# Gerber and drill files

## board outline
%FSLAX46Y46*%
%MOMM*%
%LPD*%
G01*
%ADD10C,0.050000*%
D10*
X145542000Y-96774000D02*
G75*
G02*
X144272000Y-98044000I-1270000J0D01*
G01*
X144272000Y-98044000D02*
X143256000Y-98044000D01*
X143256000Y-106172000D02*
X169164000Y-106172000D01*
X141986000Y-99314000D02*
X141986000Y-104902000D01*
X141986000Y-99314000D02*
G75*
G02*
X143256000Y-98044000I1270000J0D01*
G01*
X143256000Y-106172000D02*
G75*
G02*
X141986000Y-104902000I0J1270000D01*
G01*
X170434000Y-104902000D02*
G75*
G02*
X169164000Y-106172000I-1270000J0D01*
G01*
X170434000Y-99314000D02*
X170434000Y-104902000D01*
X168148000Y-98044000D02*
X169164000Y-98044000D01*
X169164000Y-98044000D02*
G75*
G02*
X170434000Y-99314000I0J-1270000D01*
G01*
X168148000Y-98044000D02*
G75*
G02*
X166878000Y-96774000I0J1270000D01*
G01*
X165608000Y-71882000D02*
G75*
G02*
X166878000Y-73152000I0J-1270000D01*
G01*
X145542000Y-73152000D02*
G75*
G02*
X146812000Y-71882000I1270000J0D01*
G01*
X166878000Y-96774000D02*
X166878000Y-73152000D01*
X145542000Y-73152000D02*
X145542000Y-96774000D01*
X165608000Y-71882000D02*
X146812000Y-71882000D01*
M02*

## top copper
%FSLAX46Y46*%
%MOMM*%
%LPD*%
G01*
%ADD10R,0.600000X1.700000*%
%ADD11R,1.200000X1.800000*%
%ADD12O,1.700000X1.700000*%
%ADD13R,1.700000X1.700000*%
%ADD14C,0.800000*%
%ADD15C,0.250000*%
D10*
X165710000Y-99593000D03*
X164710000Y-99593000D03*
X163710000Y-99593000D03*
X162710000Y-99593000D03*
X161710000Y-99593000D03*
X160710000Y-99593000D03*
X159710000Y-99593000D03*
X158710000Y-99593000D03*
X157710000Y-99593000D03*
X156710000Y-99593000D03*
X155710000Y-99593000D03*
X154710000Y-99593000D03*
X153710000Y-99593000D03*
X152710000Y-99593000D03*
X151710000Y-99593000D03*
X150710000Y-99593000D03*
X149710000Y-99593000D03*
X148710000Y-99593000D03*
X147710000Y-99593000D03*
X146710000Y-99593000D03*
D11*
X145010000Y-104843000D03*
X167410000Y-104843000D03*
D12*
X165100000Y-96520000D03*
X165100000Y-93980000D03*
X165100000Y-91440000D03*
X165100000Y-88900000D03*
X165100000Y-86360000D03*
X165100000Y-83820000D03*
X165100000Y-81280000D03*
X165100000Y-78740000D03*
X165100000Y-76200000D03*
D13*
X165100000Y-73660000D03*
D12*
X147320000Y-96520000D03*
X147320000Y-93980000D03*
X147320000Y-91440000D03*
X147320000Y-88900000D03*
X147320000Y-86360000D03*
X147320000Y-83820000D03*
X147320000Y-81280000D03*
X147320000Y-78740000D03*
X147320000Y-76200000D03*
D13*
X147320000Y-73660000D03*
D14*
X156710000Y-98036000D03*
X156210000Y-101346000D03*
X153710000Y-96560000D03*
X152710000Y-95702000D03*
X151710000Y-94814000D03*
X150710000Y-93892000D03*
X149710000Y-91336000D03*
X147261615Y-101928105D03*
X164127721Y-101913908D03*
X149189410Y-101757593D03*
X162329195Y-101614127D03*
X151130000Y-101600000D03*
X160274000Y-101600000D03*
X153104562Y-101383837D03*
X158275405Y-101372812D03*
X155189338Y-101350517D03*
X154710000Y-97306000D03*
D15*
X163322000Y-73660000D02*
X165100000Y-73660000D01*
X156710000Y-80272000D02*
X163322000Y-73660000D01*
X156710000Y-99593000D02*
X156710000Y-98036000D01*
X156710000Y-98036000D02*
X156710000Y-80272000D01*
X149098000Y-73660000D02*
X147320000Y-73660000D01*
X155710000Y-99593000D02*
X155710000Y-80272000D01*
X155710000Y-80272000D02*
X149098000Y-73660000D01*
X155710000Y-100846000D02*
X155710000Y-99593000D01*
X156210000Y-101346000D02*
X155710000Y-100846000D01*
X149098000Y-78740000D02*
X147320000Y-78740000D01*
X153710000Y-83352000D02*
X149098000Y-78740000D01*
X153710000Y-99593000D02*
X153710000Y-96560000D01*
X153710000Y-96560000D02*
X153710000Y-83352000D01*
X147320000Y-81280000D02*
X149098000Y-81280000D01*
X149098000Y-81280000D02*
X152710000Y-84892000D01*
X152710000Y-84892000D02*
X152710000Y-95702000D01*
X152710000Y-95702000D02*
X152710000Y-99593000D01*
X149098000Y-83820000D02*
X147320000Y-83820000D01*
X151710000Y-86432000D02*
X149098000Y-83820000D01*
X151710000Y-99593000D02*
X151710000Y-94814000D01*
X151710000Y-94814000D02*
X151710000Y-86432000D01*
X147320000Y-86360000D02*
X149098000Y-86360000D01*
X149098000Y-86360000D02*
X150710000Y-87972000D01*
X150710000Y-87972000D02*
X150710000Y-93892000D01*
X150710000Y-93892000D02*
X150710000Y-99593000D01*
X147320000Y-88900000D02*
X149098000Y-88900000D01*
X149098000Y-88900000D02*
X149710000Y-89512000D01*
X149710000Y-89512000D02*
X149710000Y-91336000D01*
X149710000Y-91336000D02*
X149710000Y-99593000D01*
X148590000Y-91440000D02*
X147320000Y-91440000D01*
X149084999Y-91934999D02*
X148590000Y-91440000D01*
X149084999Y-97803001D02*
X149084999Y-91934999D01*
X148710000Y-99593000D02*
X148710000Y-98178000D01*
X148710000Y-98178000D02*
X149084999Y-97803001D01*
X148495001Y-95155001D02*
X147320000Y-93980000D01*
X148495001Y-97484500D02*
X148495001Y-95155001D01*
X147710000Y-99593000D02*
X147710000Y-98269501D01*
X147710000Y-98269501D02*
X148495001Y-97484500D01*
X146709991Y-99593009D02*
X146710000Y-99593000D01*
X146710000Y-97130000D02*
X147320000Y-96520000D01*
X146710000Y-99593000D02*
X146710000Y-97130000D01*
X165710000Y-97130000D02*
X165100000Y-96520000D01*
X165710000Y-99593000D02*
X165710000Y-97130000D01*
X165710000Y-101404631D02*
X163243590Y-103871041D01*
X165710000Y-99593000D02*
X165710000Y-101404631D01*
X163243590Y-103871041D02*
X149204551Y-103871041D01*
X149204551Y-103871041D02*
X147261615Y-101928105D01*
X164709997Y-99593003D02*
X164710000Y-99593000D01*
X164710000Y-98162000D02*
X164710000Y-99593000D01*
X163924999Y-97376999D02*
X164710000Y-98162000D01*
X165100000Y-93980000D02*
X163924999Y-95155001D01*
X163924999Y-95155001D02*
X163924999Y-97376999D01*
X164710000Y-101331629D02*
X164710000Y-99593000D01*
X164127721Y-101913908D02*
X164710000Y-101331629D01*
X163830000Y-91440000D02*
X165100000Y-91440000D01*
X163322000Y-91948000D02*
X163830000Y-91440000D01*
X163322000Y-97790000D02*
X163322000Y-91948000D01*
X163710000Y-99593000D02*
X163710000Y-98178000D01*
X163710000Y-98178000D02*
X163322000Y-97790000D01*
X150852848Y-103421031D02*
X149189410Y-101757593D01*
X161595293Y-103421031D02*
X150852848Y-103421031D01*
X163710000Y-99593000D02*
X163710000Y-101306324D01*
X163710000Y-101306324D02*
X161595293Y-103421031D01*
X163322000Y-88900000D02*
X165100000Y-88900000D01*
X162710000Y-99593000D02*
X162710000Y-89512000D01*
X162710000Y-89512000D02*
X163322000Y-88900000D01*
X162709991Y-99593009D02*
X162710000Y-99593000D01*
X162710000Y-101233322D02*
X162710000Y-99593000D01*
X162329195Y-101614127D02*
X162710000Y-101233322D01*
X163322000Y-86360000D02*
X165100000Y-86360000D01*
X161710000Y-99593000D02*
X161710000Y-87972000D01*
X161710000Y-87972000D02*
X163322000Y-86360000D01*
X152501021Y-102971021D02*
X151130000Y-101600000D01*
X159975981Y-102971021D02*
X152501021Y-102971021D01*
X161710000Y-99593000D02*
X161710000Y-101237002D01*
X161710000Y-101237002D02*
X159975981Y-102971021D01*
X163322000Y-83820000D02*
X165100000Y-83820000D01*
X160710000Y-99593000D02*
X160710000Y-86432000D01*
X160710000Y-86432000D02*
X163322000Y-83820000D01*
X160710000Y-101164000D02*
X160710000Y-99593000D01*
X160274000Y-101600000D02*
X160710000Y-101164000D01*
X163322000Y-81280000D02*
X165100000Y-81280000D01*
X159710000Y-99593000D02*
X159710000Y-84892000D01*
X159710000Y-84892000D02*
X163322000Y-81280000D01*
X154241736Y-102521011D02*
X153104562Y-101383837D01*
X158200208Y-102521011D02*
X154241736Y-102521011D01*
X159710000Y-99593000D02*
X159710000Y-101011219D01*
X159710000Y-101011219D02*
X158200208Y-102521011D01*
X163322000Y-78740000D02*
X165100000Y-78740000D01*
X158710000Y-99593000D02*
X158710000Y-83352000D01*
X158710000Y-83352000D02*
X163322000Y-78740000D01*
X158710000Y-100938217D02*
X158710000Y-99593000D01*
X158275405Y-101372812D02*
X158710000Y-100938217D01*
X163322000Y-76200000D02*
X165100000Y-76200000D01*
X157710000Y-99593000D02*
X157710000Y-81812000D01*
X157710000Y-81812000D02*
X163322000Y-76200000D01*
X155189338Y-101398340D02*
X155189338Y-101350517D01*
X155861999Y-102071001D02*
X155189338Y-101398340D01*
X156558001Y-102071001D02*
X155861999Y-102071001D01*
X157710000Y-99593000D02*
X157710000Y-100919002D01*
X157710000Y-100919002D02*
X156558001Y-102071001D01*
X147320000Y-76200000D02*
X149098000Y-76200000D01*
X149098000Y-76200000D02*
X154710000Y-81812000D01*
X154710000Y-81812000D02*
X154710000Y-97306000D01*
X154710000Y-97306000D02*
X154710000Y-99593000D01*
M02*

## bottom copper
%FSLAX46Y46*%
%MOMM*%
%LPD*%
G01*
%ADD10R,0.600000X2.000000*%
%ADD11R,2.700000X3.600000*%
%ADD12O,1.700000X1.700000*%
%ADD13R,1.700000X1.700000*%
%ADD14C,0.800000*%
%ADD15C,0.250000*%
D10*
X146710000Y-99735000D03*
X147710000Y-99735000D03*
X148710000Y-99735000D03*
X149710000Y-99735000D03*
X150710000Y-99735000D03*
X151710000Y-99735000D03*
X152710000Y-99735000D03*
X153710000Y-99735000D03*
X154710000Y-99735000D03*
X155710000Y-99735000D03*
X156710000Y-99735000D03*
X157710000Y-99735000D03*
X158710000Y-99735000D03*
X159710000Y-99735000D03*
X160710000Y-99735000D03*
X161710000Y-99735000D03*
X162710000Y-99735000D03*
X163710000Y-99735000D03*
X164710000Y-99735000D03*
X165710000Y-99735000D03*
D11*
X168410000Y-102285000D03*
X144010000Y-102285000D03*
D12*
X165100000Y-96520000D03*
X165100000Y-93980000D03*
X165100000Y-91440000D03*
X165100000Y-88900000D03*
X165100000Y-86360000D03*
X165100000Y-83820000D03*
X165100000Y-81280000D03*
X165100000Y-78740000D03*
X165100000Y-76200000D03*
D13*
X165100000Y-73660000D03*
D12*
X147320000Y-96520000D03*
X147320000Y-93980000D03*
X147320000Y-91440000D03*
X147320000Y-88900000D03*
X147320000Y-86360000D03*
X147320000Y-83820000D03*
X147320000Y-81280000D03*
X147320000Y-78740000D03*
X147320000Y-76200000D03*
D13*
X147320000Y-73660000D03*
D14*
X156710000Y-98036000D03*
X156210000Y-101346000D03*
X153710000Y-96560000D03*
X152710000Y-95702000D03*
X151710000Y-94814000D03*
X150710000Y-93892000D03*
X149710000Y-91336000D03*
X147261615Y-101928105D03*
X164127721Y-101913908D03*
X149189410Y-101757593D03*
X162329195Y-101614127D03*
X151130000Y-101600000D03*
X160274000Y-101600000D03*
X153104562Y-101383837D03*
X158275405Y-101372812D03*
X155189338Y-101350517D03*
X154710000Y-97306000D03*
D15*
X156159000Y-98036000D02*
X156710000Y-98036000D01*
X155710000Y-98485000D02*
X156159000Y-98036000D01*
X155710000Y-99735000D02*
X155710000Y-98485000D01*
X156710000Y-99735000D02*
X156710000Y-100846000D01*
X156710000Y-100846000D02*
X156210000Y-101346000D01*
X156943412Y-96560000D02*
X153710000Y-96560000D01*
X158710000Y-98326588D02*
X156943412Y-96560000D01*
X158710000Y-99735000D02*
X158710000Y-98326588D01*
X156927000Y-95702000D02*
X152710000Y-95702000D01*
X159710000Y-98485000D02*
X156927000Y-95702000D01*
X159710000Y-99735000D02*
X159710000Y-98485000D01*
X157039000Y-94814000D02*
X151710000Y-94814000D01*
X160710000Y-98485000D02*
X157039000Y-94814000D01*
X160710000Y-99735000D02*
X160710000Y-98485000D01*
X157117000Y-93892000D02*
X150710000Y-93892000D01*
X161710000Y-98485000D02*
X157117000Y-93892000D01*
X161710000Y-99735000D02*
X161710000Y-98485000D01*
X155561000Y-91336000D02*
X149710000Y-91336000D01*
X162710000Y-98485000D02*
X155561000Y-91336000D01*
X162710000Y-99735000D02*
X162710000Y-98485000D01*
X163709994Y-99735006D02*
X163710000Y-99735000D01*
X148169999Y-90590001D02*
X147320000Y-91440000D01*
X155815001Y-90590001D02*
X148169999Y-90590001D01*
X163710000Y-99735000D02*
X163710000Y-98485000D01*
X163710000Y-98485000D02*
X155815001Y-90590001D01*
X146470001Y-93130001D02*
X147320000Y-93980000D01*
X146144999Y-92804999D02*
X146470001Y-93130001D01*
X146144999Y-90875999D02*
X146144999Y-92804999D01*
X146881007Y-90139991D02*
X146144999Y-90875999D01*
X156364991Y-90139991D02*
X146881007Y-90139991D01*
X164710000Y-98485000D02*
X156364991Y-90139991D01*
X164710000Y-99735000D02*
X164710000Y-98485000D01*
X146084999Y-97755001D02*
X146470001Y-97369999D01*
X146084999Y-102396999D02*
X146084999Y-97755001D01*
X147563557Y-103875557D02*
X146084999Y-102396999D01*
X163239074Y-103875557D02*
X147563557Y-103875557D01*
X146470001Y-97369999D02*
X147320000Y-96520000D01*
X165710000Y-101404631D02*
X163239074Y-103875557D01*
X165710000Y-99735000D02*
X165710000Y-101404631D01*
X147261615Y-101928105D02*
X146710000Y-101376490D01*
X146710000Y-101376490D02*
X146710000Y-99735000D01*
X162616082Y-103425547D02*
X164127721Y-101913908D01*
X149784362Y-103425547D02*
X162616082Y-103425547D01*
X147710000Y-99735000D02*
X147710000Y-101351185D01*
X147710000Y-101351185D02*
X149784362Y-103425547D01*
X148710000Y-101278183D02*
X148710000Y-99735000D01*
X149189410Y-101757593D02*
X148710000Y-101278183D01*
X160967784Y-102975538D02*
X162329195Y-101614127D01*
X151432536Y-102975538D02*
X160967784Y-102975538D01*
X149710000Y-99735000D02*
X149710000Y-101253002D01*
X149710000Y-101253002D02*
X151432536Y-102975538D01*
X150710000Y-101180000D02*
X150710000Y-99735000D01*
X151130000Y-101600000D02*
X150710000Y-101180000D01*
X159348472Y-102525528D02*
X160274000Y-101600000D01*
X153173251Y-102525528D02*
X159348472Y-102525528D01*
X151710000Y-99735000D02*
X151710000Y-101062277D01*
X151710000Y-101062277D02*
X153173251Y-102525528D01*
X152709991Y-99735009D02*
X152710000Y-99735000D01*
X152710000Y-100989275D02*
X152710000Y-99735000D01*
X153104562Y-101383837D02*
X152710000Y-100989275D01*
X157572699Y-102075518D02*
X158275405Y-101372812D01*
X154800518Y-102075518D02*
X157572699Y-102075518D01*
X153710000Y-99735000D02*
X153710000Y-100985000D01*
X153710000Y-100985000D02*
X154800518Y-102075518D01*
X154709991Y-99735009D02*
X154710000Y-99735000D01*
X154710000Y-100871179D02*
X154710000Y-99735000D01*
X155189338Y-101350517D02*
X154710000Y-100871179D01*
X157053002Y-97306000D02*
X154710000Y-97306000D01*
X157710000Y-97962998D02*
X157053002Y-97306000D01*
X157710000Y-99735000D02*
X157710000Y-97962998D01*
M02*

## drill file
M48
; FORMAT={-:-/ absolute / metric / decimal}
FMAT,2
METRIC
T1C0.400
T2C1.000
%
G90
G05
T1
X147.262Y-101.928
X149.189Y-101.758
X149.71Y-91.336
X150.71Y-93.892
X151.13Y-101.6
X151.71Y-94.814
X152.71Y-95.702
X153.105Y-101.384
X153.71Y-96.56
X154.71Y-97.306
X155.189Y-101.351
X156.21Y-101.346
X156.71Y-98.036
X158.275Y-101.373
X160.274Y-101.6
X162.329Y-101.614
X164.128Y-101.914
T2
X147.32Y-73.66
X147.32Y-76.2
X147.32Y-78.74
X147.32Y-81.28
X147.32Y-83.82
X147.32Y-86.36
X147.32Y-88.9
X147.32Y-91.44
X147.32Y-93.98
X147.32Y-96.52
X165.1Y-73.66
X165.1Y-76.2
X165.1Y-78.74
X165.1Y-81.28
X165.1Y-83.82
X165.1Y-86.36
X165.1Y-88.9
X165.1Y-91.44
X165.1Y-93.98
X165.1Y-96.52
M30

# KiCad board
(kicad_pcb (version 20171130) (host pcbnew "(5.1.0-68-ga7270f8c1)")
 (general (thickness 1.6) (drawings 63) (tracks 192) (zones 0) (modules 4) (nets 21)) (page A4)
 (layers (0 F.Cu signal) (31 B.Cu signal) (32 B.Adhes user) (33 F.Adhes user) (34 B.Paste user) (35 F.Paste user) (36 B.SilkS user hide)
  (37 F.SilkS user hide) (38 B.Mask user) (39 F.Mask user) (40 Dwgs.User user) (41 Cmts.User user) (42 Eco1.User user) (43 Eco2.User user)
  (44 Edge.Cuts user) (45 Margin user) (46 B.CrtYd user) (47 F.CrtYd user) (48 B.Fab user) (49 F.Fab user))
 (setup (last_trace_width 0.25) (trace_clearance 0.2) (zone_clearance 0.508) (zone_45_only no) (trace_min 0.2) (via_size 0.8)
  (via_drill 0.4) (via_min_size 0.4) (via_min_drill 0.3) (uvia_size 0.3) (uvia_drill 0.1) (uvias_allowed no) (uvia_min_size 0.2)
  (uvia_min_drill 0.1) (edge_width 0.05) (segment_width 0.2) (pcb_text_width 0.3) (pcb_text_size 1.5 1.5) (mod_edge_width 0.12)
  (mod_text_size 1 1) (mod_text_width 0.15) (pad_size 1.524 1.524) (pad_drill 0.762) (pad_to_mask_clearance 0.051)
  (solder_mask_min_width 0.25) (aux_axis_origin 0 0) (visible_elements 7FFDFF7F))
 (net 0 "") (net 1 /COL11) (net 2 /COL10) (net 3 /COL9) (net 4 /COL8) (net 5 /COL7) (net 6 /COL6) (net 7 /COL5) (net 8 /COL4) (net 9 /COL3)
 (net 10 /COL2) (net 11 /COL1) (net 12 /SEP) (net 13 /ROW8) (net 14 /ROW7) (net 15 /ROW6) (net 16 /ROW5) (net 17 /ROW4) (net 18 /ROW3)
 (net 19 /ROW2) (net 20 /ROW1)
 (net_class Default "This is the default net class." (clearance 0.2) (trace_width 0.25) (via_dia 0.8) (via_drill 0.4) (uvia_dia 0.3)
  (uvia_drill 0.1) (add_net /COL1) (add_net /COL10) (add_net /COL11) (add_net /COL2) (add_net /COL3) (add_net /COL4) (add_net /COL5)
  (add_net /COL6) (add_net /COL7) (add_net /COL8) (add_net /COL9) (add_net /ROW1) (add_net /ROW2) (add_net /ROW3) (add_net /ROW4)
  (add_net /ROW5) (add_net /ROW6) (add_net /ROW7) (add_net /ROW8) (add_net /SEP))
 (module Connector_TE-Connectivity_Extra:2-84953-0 (layer B.Cu) (at 156.21 101.635 180)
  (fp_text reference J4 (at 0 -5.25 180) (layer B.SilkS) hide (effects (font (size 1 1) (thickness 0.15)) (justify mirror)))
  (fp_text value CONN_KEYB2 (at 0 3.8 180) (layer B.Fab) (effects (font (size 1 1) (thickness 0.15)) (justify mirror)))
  (pad 20 smd rect (at 9.5 1.9 180) (size 0.6 2) (layers B.Cu B.Paste B.Mask) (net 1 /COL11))
  (pad 19 smd rect (at 8.5 1.9 180) (size 0.6 2) (layers B.Cu B.Paste B.Mask) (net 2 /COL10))
  (pad 18 smd rect (at 7.5 1.9 180) (size 0.6 2) (layers B.Cu B.Paste B.Mask) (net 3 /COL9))
  (pad 17 smd rect (at 6.5 1.9 180) (size 0.6 2) (layers B.Cu B.Paste B.Mask) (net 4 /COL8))
  (pad 16 smd rect (at 5.5 1.9 180) (size 0.6 2) (layers B.Cu B.Paste B.Mask) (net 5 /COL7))
  (pad 15 smd rect (at 4.5 1.9 180) (size 0.6 2) (layers B.Cu B.Paste B.Mask) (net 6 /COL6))
  (pad 14 smd rect (at 3.5 1.9 180) (size 0.6 2) (layers B.Cu B.Paste B.Mask) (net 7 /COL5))
  (pad 13 smd rect (at 2.5 1.9 180) (size 0.6 2) (layers B.Cu B.Paste B.Mask) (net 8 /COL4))
  (pad 12 smd rect (at 1.5 1.9 180) (size 0.6 2) (layers B.Cu B.Paste B.Mask) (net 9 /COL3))
  (pad 11 smd rect (at 0.5 1.9 180) (size 0.6 2) (layers B.Cu B.Paste B.Mask) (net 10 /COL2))
  (pad 10 smd rect (at -0.5 1.9 180) (size 0.6 2) (layers B.Cu B.Paste B.Mask) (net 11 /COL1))
  (pad 9 smd rect (at -1.5 1.9 180) (size 0.6 2) (layers B.Cu B.Paste B.Mask) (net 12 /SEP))
  (pad 8 smd rect (at -2.5 1.9 180) (size 0.6 2) (layers B.Cu B.Paste B.Mask) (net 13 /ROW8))
  (pad 7 smd rect (at -3.5 1.9 180) (size 0.6 2) (layers B.Cu B.Paste B.Mask) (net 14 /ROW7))
  (pad 6 smd rect (at -4.5 1.9 180) (size 0.6 2) (layers B.Cu B.Paste B.Mask) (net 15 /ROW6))
  (pad 5 smd rect (at -5.5 1.9 180) (size 0.6 2) (layers B.Cu B.Paste B.Mask) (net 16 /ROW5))
  (pad 4 smd rect (at -6.5 1.9 180) (size 0.6 2) (layers B.Cu B.Paste B.Mask) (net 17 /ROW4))
  (pad 3 smd rect (at -7.5 1.9 180) (size 0.6 2) (layers B.Cu B.Paste B.Mask) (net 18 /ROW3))
  (pad 2 smd rect (at -8.5 1.9 180) (size 0.6 2) (layers B.Cu B.Paste B.Mask) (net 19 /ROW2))
  (pad 1 smd rect (at -9.5 1.9 180) (size 0.6 2) (layers B.Cu B.Paste B.Mask) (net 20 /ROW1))
  (pad "" smd rect (at -12.2 -0.65 180) (size 2.7 3.6) (layers B.Cu B.Paste B.Mask))
  (pad "" smd rect (at 12.2 -0.65 180) (size 2.7 3.6) (layers B.Cu B.Paste B.Mask)))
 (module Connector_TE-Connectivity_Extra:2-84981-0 (layer F.Cu) (at 156.21 102.743)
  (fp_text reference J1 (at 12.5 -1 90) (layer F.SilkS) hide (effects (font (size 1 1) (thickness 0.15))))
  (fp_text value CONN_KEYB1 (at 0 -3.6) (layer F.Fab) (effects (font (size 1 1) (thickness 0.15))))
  (pad 20 smd rect (at 9.5 -3.15) (size 0.6 1.7) (layers F.Cu F.Paste F.Mask) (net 1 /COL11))
  (pad 19 smd rect (at 8.5 -3.15) (size 0.6 1.7) (layers F.Cu F.Paste F.Mask) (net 2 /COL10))
  (pad 18 smd rect (at 7.5 -3.15) (size 0.6 1.7) (layers F.Cu F.Paste F.Mask) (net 3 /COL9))
  (pad 17 smd rect (at 6.5 -3.15) (size 0.6 1.7) (layers F.Cu F.Paste F.Mask) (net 4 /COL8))
  (pad 16 smd rect (at 5.5 -3.15) (size 0.6 1.7) (layers F.Cu F.Paste F.Mask) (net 5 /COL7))
  (pad 15 smd rect (at 4.5 -3.15) (size 0.6 1.7) (layers F.Cu F.Paste F.Mask) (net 6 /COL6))
  (pad 14 smd rect (at 3.5 -3.15) (size 0.6 1.7) (layers F.Cu F.Paste F.Mask) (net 7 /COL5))
  (pad 13 smd rect (at 2.5 -3.15) (size 0.6 1.7) (layers F.Cu F.Paste F.Mask) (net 8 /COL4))
  (pad 12 smd rect (at 1.5 -3.15) (size 0.6 1.7) (layers F.Cu F.Paste F.Mask) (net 9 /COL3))
  (pad 11 smd rect (at 0.5 -3.15) (size 0.6 1.7) (layers F.Cu F.Paste F.Mask) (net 10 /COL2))
  (pad 10 smd rect (at -0.5 -3.15) (size 0.6 1.7) (layers F.Cu F.Paste F.Mask) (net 11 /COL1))
  (pad 9 smd rect (at -1.5 -3.15) (size 0.6 1.7) (layers F.Cu F.Paste F.Mask) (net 12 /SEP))
  (pad 8 smd rect (at -2.5 -3.15) (size 0.6 1.7) (layers F.Cu F.Paste F.Mask) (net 13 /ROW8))
  (pad 7 smd rect (at -3.5 -3.15) (size 0.6 1.7) (layers F.Cu F.Paste F.Mask) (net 14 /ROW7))
  (pad 6 smd rect (at -4.5 -3.15) (size 0.6 1.7) (layers F.Cu F.Paste F.Mask) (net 15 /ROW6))
  (pad 5 smd rect (at -5.5 -3.15) (size 0.6 1.7) (layers F.Cu F.Paste F.Mask) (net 16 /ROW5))
  (pad 4 smd rect (at -6.5 -3.15) (size 0.6 1.7) (layers F.Cu F.Paste F.Mask) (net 17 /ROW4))
  (pad 3 smd rect (at -7.5 -3.15) (size 0.6 1.7) (layers F.Cu F.Paste F.Mask) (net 18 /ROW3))
  (pad 2 smd rect (at -8.5 -3.15) (size 0.6 1.7) (layers F.Cu F.Paste F.Mask) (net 19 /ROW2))
  (pad 1 smd rect (at -9.5 -3.15) (size 0.6 1.7) (layers F.Cu F.Paste F.Mask) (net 20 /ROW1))
  (pad "" smd rect (at -11.2 2.1) (size 1.2 1.8) (layers F.Cu F.Paste F.Mask))
  (pad "" smd rect (at 11.2 2.1) (size 1.2 1.8) (layers F.Cu F.Paste F.Mask)))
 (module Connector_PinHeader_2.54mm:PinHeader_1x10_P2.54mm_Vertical (layer F.Cu) (at 165.1 73.66)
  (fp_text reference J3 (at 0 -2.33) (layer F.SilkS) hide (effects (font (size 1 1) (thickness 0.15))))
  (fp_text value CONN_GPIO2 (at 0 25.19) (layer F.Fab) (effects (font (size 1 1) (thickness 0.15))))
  (pad 10 thru_hole oval (at 0 22.86) (size 1.7 1.7) (drill 1) (layers *.Cu *.Mask) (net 1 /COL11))
  (pad 9 thru_hole oval (at 0 20.32) (size 1.7 1.7) (drill 1) (layers *.Cu *.Mask) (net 2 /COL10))
  (pad 8 thru_hole oval (at 0 17.78) (size 1.7 1.7) (drill 1) (layers *.Cu *.Mask) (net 3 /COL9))
  (pad 7 thru_hole oval (at 0 15.24) (size 1.7 1.7) (drill 1) (layers *.Cu *.Mask) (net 4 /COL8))
  (pad 6 thru_hole oval (at 0 12.7) (size 1.7 1.7) (drill 1) (layers *.Cu *.Mask) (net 5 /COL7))
  (pad 5 thru_hole oval (at 0 10.16) (size 1.7 1.7) (drill 1) (layers *.Cu *.Mask) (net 6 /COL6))
  (pad 4 thru_hole oval (at 0 7.62) (size 1.7 1.7) (drill 1) (layers *.Cu *.Mask) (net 7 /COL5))
  (pad 3 thru_hole oval (at 0 5.08) (size 1.7 1.7) (drill 1) (layers *.Cu *.Mask) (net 8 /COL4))
  (pad 2 thru_hole oval (at 0 2.54) (size 1.7 1.7) (drill 1) (layers *.Cu *.Mask) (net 9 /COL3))
  (pad 1 thru_hole rect (at 0 0) (size 1.7 1.7) (drill 1) (layers *.Cu *.Mask) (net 10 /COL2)))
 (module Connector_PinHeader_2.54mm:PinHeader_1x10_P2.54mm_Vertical (layer F.Cu) (at 147.32 73.66)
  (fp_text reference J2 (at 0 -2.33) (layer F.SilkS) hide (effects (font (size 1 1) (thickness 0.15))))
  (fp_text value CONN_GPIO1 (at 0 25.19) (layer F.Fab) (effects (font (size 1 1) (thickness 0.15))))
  (pad 10 thru_hole oval (at 0 22.86) (size 1.7 1.7) (drill 1) (layers *.Cu *.Mask) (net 20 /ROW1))
  (pad 9 thru_hole oval (at 0 20.32) (size 1.7 1.7) (drill 1) (layers *.Cu *.Mask) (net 19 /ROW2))
  (pad 8 thru_hole oval (at 0 17.78) (size 1.7 1.7) (drill 1) (layers *.Cu *.Mask) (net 18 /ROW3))
  (pad 7 thru_hole oval (at 0 15.24) (size 1.7 1.7) (drill 1) (layers *.Cu *.Mask) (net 17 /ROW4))
  (pad 6 thru_hole oval (at 0 12.7) (size 1.7 1.7) (drill 1) (layers *.Cu *.Mask) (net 16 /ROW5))
  (pad 5 thru_hole oval (at 0 10.16) (size 1.7 1.7) (drill 1) (layers *.Cu *.Mask) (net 15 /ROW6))
  (pad 4 thru_hole oval (at 0 7.62) (size 1.7 1.7) (drill 1) (layers *.Cu *.Mask) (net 14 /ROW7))
  (pad 3 thru_hole oval (at 0 5.08) (size 1.7 1.7) (drill 1) (layers *.Cu *.Mask) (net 13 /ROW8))
  (pad 2 thru_hole oval (at 0 2.54) (size 1.7 1.7) (drill 1) (layers *.Cu *.Mask) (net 12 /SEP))
  (pad 1 thru_hole rect (at 0 0) (size 1.7 1.7) (drill 1) (layers *.Cu *.Mask) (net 11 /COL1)))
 (gr_arc (start 144.272 96.774) (end 144.272 98.044) (angle -90) (layer Edge.Cuts) (width 0.05))
 (gr_line (start 144.272 98.044) (end 143.256 98.044) (layer Edge.Cuts) (width 0.05))
 (gr_line (start 143.256 106.172) (end 169.164 106.172) (layer Edge.Cuts) (width 0.05))
 (gr_line (start 141.986 99.314) (end 141.986 104.902) (layer Edge.Cuts) (width 0.05))
 (gr_arc (start 143.256 99.314) (end 143.256 98.044) (angle -90) (layer Edge.Cuts) (width 0.05))
 (gr_arc (start 143.256 104.902) (end 141.986 104.902) (angle -90) (layer Edge.Cuts) (width 0.05))
 (gr_arc (start 169.164 104.902) (end 169.164 106.172) (angle -90) (layer Edge.Cuts) (width 0.05))
 (gr_line (start 170.434 99.314) (end 170.434 104.902) (layer Edge.Cuts) (width 0.05))
 (gr_line (start 168.148 98.044) (end 169.164 98.044) (layer Edge.Cuts) (width 0.05))
 (gr_arc (start 169.164 99.314) (end 170.434 99.314) (angle -90) (layer Edge.Cuts) (width 0.05))
 (gr_arc (start 168.148 96.774) (end 166.878 96.774) (angle -90) (layer Edge.Cuts) (width 0.05))
 (gr_arc (start 165.608 73.152) (end 166.878 73.152) (angle -90) (layer Edge.Cuts) (width 0.05))
 (gr_arc (start 146.812 73.152) (end 146.812 71.882) (angle -90) (layer Edge.Cuts) (width 0.05))
 (gr_line (start 166.878 96.774) (end 166.878 73.152) (layer Edge.Cuts) (width 0.05))
 (gr_line (start 145.542 73.152) (end 145.542 96.774) (layer Edge.Cuts) (width 0.05))
 (gr_line (start 165.608 71.882) (end 146.812 71.882) (layer Edge.Cuts) (width 0.05))
 (segment (start 163.322 73.66) (end 165.1 73.66) (width 0.25) (layer F.Cu) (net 10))
 (segment (start 156.71 80.272) (end 163.322 73.66) (width 0.25) (layer F.Cu) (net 10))
 (via (at 156.71 98.036) (size 0.8) (drill 0.4) (layers F.Cu B.Cu) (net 10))
 (segment (start 156.159 98.036) (end 156.71 98.036) (width 0.25) (layer B.Cu) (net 10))
 (segment (start 155.71 98.485) (end 156.159 98.036) (width 0.25) (layer B.Cu) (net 10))
 (segment (start 155.71 99.735) (end 155.71 98.485) (width 0.25) (layer B.Cu) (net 10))
 (segment (start 156.71 99.593) (end 156.71 98.036) (width 0.25) (layer F.Cu) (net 10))
 (segment (start 156.71 98.036) (end 156.71 80.272) (width 0.25) (layer F.Cu) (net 10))
 (segment (start 149.098 73.66) (end 147.32 73.66) (width 0.25) (layer F.Cu) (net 11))
 (segment (start 155.71 99.593) (end 155.71 80.272) (width 0.25) (layer F.Cu) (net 11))
 (segment (start 155.71 80.272) (end 149.098 73.66) (width 0.25) (layer F.Cu) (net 11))
 (via (at 156.21 101.346) (size 0.8) (drill 0.4) (layers F.Cu B.Cu) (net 11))
 (segment (start 156.71 99.735) (end 156.71 100.846) (width 0.25) (layer B.Cu) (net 11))
 (segment (start 156.71 100.846) (end 156.21 101.346) (width 0.25) (layer B.Cu) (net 11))
 (segment (start 155.71 100.846) (end 155.71 99.593) (width 0.25) (layer F.Cu) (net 11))
 (segment (start 156.21 101.346) (end 155.71 100.846) (width 0.25) (layer F.Cu) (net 11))
 (segment (start 149.098 78.74) (end 147.32 78.74) (width 0.25) (layer F.Cu) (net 13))
 (segment (start 153.71 83.352) (end 149.098 78.74) (width 0.25) (layer F.Cu) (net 13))
 (via (at 153.71 96.56) (size 0.8) (drill 0.4) (layers F.Cu B.Cu) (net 13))
 (segment (start 156.943412 96.56) (end 153.71 96.56) (width 0.25) (layer B.Cu) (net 13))
 (segment (start 158.71 98.326588) (end 156.943412 96.56) (width 0.25) (layer B.Cu) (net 13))
 (segment (start 158.71 99.735) (end 158.71 98.326588) (width 0.25) (layer B.Cu) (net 13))
 (segment (start 153.71 99.593) (end 153.71 96.56) (width 0.25) (layer F.Cu) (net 13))
 (segment (start 153.71 96.56) (end 153.71 83.352) (width 0.25) (layer F.Cu) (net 13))
 (segment (start 147.32 81.28) (end 149.098 81.28) (width 0.25) (layer F.Cu) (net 14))
 (segment (start 149.098 81.28) (end 152.71 84.892) (width 0.25) (layer F.Cu) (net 14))
 (via (at 152.71 95.702) (size 0.8) (drill 0.4) (layers F.Cu B.Cu) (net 14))
 (segment (start 156.927 95.702) (end 152.71 95.702) (width 0.25) (layer B.Cu) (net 14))
 (segment (start 159.71 98.485) (end 156.927 95.702) (width 0.25) (layer B.Cu) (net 14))
 (segment (start 159.71 99.735) (end 159.71 98.485) (width 0.25) (layer B.Cu) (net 14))
 (segment (start 152.71 84.892) (end 152.71 95.702) (width 0.25) (layer F.Cu) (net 14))
 (segment (start 152.71 95.702) (end 152.71 99.593) (width 0.25) (layer F.Cu) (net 14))
 (segment (start 149.098 83.82) (end 147.32 83.82) (width 0.25) (layer F.Cu) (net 15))
 (segment (start 151.71 86.432) (end 149.098 83.82) (width 0.25) (layer F.Cu) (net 15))
 (via (at 151.71 94.814) (size 0.8) (drill 0.4) (layers F.Cu B.Cu) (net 15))
 (segment (start 157.039 94.814) (end 151.71 94.814) (width 0.25) (layer B.Cu) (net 15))
 (segment (start 160.71 98.485) (end 157.039 94.814) (width 0.25) (layer B.Cu) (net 15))
 (segment (start 160.71 99.735) (end 160.71 98.485) (width 0.25) (layer B.Cu) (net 15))
 (segment (start 151.71 99.593) (end 151.71 94.814) (width 0.25) (layer F.Cu) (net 15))
 (segment (start 151.71 94.814) (end 151.71 86.432) (width 0.25) (layer F.Cu) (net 15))
 (segment (start 147.32 86.36) (end 149.098 86.36) (width 0.25) (layer F.Cu) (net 16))
 (segment (start 149.098 86.36) (end 150.71 87.972) (width 0.25) (layer F.Cu) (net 16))
 (via (at 150.71 93.892) (size 0.8) (drill 0.4) (layers F.Cu B.Cu) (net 16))
 (segment (start 157.117 93.892) (end 150.71 93.892) (width 0.25) (layer B.Cu) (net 16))
 (segment (start 161.71 98.485) (end 157.117 93.892) (width 0.25) (layer B.Cu) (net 16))
 (segment (start 161.71 99.735) (end 161.71 98.485) (width 0.25) (layer B.Cu) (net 16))
 (segment (start 150.71 87.972) (end 150.71 93.892) (width 0.25) (layer F.Cu) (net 16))
 (segment (start 150.71 93.892) (end 150.71 99.593) (width 0.25) (layer F.Cu) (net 16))
 (segment (start 147.32 88.9) (end 149.098 88.9) (width 0.25) (layer F.Cu) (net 17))
 (segment (start 149.098 88.9) (end 149.71 89.512) (width 0.25) (layer F.Cu) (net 17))
 (via (at 149.71 91.336) (size 0.8) (drill 0.4) (layers F.Cu B.Cu) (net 17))
 (segment (start 155.561 91.336) (end 149.71 91.336) (width 0.25) (layer B.Cu) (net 17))
 (segment (start 162.71 98.485) (end 155.561 91.336) (width 0.25) (layer B.Cu) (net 17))
 (segment (start 162.71 99.735) (end 162.71 98.485) (width 0.25) (layer B.Cu) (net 17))
 (segment (start 149.71 89.512) (end 149.71 91.336) (width 0.25) (layer F.Cu) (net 17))
 (segment (start 149.71 91.336) (end 149.71 99.593) (width 0.25) (layer F.Cu) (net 17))
 (segment (start 163.709994 99.735006) (end 163.71 99.735) (width 0.25) (layer B.Cu) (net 18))
 (segment (start 148.59 91.44) (end 147.32 91.44) (width 0.25) (layer F.Cu) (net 18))
 (segment (start 149.084999 91.934999) (end 148.59 91.44) (width 0.25) (layer F.Cu) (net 18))
 (segment (start 149.084999 97.803001) (end 149.084999 91.934999) (width 0.25) (layer F.Cu) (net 18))
 (segment (start 148.71 99.593) (end 148.71 98.178) (width 0.25) (layer F.Cu) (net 18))
 (segment (start 148.71 98.178) (end 149.084999 97.803001) (width 0.25) (layer F.Cu) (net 18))
 (segment (start 148.169999 90.590001) (end 147.32 91.44) (width 0.25) (layer B.Cu) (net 18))
 (segment (start 155.815001 90.590001) (end 148.169999 90.590001) (width 0.25) (layer B.Cu) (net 18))
 (segment (start 163.71 99.735) (end 163.71 98.485) (width 0.25) (layer B.Cu) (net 18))
 (segment (start 163.71 98.485) (end 155.815001 90.590001) (width 0.25) (layer B.Cu) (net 18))
 (segment (start 148.495001 95.155001) (end 147.32 93.98) (width 0.25) (layer F.Cu) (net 19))
 (segment (start 148.495001 97.4845) (end 148.495001 95.155001) (width 0.25) (layer F.Cu) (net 19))
 (segment (start 147.71 99.593) (end 147.71 98.269501) (width 0.25) (layer F.Cu) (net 19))
 (segment (start 147.71 98.269501) (end 148.495001 97.4845) (width 0.25) (layer F.Cu) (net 19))
 (segment (start 146.470001 93.130001) (end 147.32 93.98) (width 0.25) (layer B.Cu) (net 19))
 (segment (start 146.144999 92.804999) (end 146.470001 93.130001) (width 0.25) (layer B.Cu) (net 19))
 (segment (start 146.144999 90.875999) (end 146.144999 92.804999) (width 0.25) (layer B.Cu) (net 19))
 (segment (start 146.881007 90.139991) (end 146.144999 90.875999) (width 0.25) (layer B.Cu) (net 19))
 (segment (start 156.364991 90.139991) (end 146.881007 90.139991) (width 0.25) (layer B.Cu) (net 19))
 (segment (start 164.71 98.485) (end 156.364991 90.139991) (width 0.25) (layer B.Cu) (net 19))
 (segment (start 164.71 99.735) (end 164.71 98.485) (width 0.25) (layer B.Cu) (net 19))
 (segment (start 146.709991 99.593009) (end 146.71 99.593) (width 0.25) (layer F.Cu) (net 20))
 (segment (start 146.71 97.13) (end 147.32 96.52) (width 0.25) (layer F.Cu) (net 20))
 (segment (start 146.71 99.593) (end 146.71 97.13) (width 0.25) (layer F.Cu) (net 20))
 (segment (start 146.084999 97.755001) (end 146.470001 97.369999) (width 0.25) (layer B.Cu) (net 20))
 (segment (start 146.084999 102.396999) (end 146.084999 97.755001) (width 0.25) (layer B.Cu) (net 20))
 (segment (start 147.563557 103.875557) (end 146.084999 102.396999) (width 0.25) (layer B.Cu) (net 20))
 (segment (start 163.239074 103.875557) (end 147.563557 103.875557) (width 0.25) (layer B.Cu) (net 20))
 (segment (start 146.470001 97.369999) (end 147.32 96.52) (width 0.25) (layer B.Cu) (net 20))
 (segment (start 165.71 101.404631) (end 163.239074 103.875557) (width 0.25) (layer B.Cu) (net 20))
 (segment (start 165.71 99.735) (end 165.71 101.404631) (width 0.25) (layer B.Cu) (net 20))
 (segment (start 165.71 97.13) (end 165.1 96.52) (width 0.25) (layer F.Cu) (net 1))
 (segment (start 165.71 99.593) (end 165.71 97.13) (width 0.25) (layer F.Cu) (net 1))
 (via (at 147.261615 101.928105) (size 0.8) (drill 0.4) (layers F.Cu B.Cu) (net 1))
 (segment (start 147.261615 101.928105) (end 146.71 101.37649) (width 0.25) (layer B.Cu) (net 1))
 (segment (start 146.71 101.37649) (end 146.71 99.735) (width 0.25) (layer B.Cu) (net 1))
 (segment (start 165.71 101.404631) (end 163.24359 103.871041) (width 0.25) (layer F.Cu) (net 1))
 (segment (start 165.71 99.593) (end 165.71 101.404631) (width 0.25) (layer F.Cu) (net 1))
 (segment (start 163.24359 103.871041) (end 149.204551 103.871041) (width 0.25) (layer F.Cu) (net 1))
 (segment (start 149.204551 103.871041) (end 147.261615 101.928105) (width 0.25) (layer F.Cu) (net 1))
 (segment (start 164.709997 99.593003) (end 164.71 99.593) (width 0.25) (layer F.Cu) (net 2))
 (segment (start 164.71 98.162) (end 164.71 99.593) (width 0.25) (layer F.Cu) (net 2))
 (segment (start 163.924999 97.376999) (end 164.71 98.162) (width 0.25) (layer F.Cu) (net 2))
 (segment (start 165.1 93.98) (end 163.924999 95.155001) (width 0.25) (layer F.Cu) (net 2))
 (segment (start 163.924999 95.155001) (end 163.924999 97.376999) (width 0.25) (layer F.Cu) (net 2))
 (via (at 164.127721 101.913908) (size 0.8) (drill 0.4) (layers F.Cu B.Cu) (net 2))
 (segment (start 162.616082 103.425547) (end 164.127721 101.913908) (width 0.25) (layer B.Cu) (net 2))
 (segment (start 149.784362 103.425547) (end 162.616082 103.425547) (width 0.25) (layer B.Cu) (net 2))
 (segment (start 147.71 99.735) (end 147.71 101.351185) (width 0.25) (layer B.Cu) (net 2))
 (segment (start 147.71 101.351185) (end 149.784362 103.425547) (width 0.25) (layer B.Cu) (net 2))
 (segment (start 164.71 101.331629) (end 164.71 99.593) (width 0.25) (layer F.Cu) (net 2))
 (segment (start 164.127721 101.913908) (end 164.71 101.331629) (width 0.25) (layer F.Cu) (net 2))
 (segment (start 163.83 91.44) (end 165.1 91.44) (width 0.25) (layer F.Cu) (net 3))
 (segment (start 163.322 91.948) (end 163.83 91.44) (width 0.25) (layer F.Cu) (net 3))
 (segment (start 163.322 97.79) (end 163.322 91.948) (width 0.25) (layer F.Cu) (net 3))
 (segment (start 163.71 99.593) (end 163.71 98.178) (width 0.25) (layer F.Cu) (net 3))
 (segment (start 163.71 98.178) (end 163.322 97.79) (width 0.25) (layer F.Cu) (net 3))
 (via (at 149.18941 101.757593) (size 0.8) (drill 0.4) (layers F.Cu B.Cu) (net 3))
 (segment (start 150.852848 103.421031) (end 149.18941 101.757593) (width 0.25) (layer F.Cu) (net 3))
 (segment (start 161.595293 103.421031) (end 150.852848 103.421031) (width 0.25) (layer F.Cu) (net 3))
 (segment (start 163.71 99.593) (end 163.71 101.306324) (width 0.25) (layer F.Cu) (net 3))
 (segment (start 163.71 101.306324) (end 161.595293 103.421031) (width 0.25) (layer F.Cu) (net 3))
 (segment (start 148.71 101.278183) (end 148.71 99.735) (width 0.25) (layer B.Cu) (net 3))
 (segment (start 149.18941 101.757593) (end 148.71 101.278183) (width 0.25) (layer B.Cu) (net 3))
 (segment (start 163.322 88.9) (end 165.1 88.9) (width 0.25) (layer F.Cu) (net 4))
 (segment (start 162.71 99.593) (end 162.71 89.512) (width 0.25) (layer F.Cu) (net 4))
 (segment (start 162.71 89.512) (end 163.322 88.9) (width 0.25) (layer F.Cu) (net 4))
 (segment (start 162.709991 99.593009) (end 162.71 99.593) (width 0.25) (layer F.Cu) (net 4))
 (via (at 162.329195 101.614127) (size 0.8) (drill 0.4) (layers F.Cu B.Cu) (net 4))
 (segment (start 160.967784 102.975538) (end 162.329195 101.614127) (width 0.25) (layer B.Cu) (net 4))
 (segment (start 151.432536 102.975538) (end 160.967784 102.975538) (width 0.25) (layer B.Cu) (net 4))
 (segment (start 149.71 99.735) (end 149.71 101.253002) (width 0.25) (layer B.Cu) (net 4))
 (segment (start 149.71 101.253002) (end 151.432536 102.975538) (width 0.25) (layer B.Cu) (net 4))
 (segment (start 162.71 101.233322) (end 162.71 99.593) (width 0.25) (layer F.Cu) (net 4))
 (segment (start 162.329195 101.614127) (end 162.71 101.233322) (width 0.25) (layer F.Cu) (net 4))
 (segment (start 163.322 86.36) (end 165.1 86.36) (width 0.25) (layer F.Cu) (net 5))
 (segment (start 161.71 99.593) (end 161.71 87.972) (width 0.25) (layer F.Cu) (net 5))
 (segment (start 161.71 87.972) (end 163.322 86.36) (width 0.25) (layer F.Cu) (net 5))
 (via (at 151.13 101.6) (size 0.8) (drill 0.4) (layers F.Cu B.Cu) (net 5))
 (segment (start 152.501021 102.971021) (end 151.13 101.6) (width 0.25) (layer F.Cu) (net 5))
 (segment (start 159.975981 102.971021) (end 152.501021 102.971021) (width 0.25) (layer F.Cu) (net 5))
 (segment (start 161.71 99.593) (end 161.71 101.237002) (width 0.25) (layer F.Cu) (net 5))
 (segment (start 161.71 101.237002) (end 159.975981 102.971021) (width 0.25) (layer F.Cu) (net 5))
 (segment (start 150.71 101.18) (end 150.71 99.735) (width 0.25) (layer B.Cu) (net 5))
 (segment (start 151.13 101.6) (end 150.71 101.18) (width 0.25) (layer B.Cu) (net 5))
 (segment (start 163.322 83.82) (end 165.1 83.82) (width 0.25) (layer F.Cu) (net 6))
 (segment (start 160.71 99.593) (end 160.71 86.432) (width 0.25) (layer F.Cu) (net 6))
 (segment (start 160.71 86.432) (end 163.322 83.82) (width 0.25) (layer F.Cu) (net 6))
 (via (at 160.274 101.6) (size 0.8) (drill 0.4) (layers F.Cu B.Cu) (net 6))
 (segment (start 159.348472 102.525528) (end 160.274 101.6) (width 0.25) (layer B.Cu) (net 6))
 (segment (start 153.173251 102.525528) (end 159.348472 102.525528) (width 0.25) (layer B.Cu) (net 6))
 (segment (start 151.71 99.735) (end 151.71 101.062277) (width 0.25) (layer B.Cu) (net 6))
 (segment (start 151.71 101.062277) (end 153.173251 102.525528) (width 0.25) (layer B.Cu) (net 6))
 (segment (start 160.71 101.164) (end 160.71 99.593) (width 0.25) (layer F.Cu) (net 6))
 (segment (start 160.274 101.6) (end 160.71 101.164) (width 0.25) (layer F.Cu) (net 6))
 (segment (start 152.709991 99.735009) (end 152.71 99.735) (width 0.25) (layer B.Cu) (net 7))
 (segment (start 163.322 81.28) (end 165.1 81.28) (width 0.25) (layer F.Cu) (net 7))
 (segment (start 159.71 99.593) (end 159.71 84.892) (width 0.25) (layer F.Cu) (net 7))
 (segment (start 159.71 84.892) (end 163.322 81.28) (width 0.25) (layer F.Cu) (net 7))
 (via (at 153.104562 101.383837) (size 0.8) (drill 0.4) (layers F.Cu B.Cu) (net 7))
 (segment (start 154.241736 102.521011) (end 153.104562 101.383837) (width 0.25) (layer F.Cu) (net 7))
 (segment (start 158.200208 102.521011) (end 154.241736 102.521011) (width 0.25) (layer F.Cu) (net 7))
 (segment (start 159.71 99.593) (end 159.71 101.011219) (width 0.25) (layer F.Cu) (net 7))
 (segment (start 159.71 101.011219) (end 158.200208 102.521011) (width 0.25) (layer F.Cu) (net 7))
 (segment (start 152.71 100.989275) (end 152.71 99.735) (width 0.25) (layer B.Cu) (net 7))
 (segment (start 153.104562 101.383837) (end 152.71 100.989275) (width 0.25) (layer B.Cu) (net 7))
 (segment (start 163.322 78.74) (end 165.1 78.74) (width 0.25) (layer F.Cu) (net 8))
 (segment (start 158.71 99.593) (end 158.71 83.352) (width 0.25) (layer F.Cu) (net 8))
 (segment (start 158.71 83.352) (end 163.322 78.74) (width 0.25) (layer F.Cu) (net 8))
 (via (at 158.275405 101.372812) (size 0.8) (drill 0.4) (layers F.Cu B.Cu) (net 8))
 (segment (start 157.572699 102.075518) (end 158.275405 101.372812) (width 0.25) (layer B.Cu) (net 8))
 (segment (start 154.800518 102.075518) (end 157.572699 102.075518) (width 0.25) (layer B.Cu) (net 8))
 (segment (start 153.71 99.735) (end 153.71 100.985) (width 0.25) (layer B.Cu) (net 8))
 (segment (start 153.71 100.985) (end 154.800518 102.075518) (width 0.25) (layer B.Cu) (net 8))
 (segment (start 158.71 100.938217) (end 158.71 99.593) (width 0.25) (layer F.Cu) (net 8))
 (segment (start 158.275405 101.372812) (end 158.71 100.938217) (width 0.25) (layer F.Cu) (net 8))
 (segment (start 163.322 76.2) (end 165.1 76.2) (width 0.25) (layer F.Cu) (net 9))
 (segment (start 157.71 99.593) (end 157.71 81.812) (width 0.25) (layer F.Cu) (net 9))
 (segment (start 157.71 81.812) (end 163.322 76.2) (width 0.25) (layer F.Cu) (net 9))
 (segment (start 154.709991 99.735009) (end 154.71 99.735) (width 0.25) (layer B.Cu) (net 9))
 (via (at 155.189338 101.350517) (size 0.8) (drill 0.4) (layers F.Cu B.Cu) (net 9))
 (segment (start 155.189338 101.39834) (end 155.189338 101.350517) (width 0.25) (layer F.Cu) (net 9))
 (segment (start 155.861999 102.071001) (end 155.189338 101.39834) (width 0.25) (layer F.Cu) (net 9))
 (segment (start 156.558001 102.071001) (end 155.861999 102.071001) (width 0.25) (layer F.Cu) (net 9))
 (segment (start 157.71 99.593) (end 157.71 100.919002) (width 0.25) (layer F.Cu) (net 9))
 (segment (start 157.71 100.919002) (end 156.558001 102.071001) (width 0.25) (layer F.Cu) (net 9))
 (segment (start 154.71 100.871179) (end 154.71 99.735) (width 0.25) (layer B.Cu) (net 9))
 (segment (start 155.189338 101.350517) (end 154.71 100.871179) (width 0.25) (layer B.Cu) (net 9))
 (segment (start 147.32 76.2) (end 149.098 76.2) (width 0.25) (layer F.Cu) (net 12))
 (segment (start 149.098 76.2) (end 154.71 81.812) (width 0.25) (layer F.Cu) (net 12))
 (via (at 154.71 97.306) (size 0.8) (drill 0.4) (layers F.Cu B.Cu) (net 12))
 (segment (start 157.053002 97.306) (end 154.71 97.306) (width 0.25) (layer B.Cu) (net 12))
 (segment (start 157.71 97.962998) (end 157.053002 97.306) (width 0.25) (layer B.Cu) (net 12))
 (segment (start 157.71 99.735) (end 157.71 97.962998) (width 0.25) (layer B.Cu) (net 12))
 (segment (start 154.71 81.812) (end 154.71 97.306) (width 0.25) (layer F.Cu) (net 12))
 (segment (start 154.71 97.306) (end 154.71 99.593) (width 0.25) (layer F.Cu) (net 12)))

